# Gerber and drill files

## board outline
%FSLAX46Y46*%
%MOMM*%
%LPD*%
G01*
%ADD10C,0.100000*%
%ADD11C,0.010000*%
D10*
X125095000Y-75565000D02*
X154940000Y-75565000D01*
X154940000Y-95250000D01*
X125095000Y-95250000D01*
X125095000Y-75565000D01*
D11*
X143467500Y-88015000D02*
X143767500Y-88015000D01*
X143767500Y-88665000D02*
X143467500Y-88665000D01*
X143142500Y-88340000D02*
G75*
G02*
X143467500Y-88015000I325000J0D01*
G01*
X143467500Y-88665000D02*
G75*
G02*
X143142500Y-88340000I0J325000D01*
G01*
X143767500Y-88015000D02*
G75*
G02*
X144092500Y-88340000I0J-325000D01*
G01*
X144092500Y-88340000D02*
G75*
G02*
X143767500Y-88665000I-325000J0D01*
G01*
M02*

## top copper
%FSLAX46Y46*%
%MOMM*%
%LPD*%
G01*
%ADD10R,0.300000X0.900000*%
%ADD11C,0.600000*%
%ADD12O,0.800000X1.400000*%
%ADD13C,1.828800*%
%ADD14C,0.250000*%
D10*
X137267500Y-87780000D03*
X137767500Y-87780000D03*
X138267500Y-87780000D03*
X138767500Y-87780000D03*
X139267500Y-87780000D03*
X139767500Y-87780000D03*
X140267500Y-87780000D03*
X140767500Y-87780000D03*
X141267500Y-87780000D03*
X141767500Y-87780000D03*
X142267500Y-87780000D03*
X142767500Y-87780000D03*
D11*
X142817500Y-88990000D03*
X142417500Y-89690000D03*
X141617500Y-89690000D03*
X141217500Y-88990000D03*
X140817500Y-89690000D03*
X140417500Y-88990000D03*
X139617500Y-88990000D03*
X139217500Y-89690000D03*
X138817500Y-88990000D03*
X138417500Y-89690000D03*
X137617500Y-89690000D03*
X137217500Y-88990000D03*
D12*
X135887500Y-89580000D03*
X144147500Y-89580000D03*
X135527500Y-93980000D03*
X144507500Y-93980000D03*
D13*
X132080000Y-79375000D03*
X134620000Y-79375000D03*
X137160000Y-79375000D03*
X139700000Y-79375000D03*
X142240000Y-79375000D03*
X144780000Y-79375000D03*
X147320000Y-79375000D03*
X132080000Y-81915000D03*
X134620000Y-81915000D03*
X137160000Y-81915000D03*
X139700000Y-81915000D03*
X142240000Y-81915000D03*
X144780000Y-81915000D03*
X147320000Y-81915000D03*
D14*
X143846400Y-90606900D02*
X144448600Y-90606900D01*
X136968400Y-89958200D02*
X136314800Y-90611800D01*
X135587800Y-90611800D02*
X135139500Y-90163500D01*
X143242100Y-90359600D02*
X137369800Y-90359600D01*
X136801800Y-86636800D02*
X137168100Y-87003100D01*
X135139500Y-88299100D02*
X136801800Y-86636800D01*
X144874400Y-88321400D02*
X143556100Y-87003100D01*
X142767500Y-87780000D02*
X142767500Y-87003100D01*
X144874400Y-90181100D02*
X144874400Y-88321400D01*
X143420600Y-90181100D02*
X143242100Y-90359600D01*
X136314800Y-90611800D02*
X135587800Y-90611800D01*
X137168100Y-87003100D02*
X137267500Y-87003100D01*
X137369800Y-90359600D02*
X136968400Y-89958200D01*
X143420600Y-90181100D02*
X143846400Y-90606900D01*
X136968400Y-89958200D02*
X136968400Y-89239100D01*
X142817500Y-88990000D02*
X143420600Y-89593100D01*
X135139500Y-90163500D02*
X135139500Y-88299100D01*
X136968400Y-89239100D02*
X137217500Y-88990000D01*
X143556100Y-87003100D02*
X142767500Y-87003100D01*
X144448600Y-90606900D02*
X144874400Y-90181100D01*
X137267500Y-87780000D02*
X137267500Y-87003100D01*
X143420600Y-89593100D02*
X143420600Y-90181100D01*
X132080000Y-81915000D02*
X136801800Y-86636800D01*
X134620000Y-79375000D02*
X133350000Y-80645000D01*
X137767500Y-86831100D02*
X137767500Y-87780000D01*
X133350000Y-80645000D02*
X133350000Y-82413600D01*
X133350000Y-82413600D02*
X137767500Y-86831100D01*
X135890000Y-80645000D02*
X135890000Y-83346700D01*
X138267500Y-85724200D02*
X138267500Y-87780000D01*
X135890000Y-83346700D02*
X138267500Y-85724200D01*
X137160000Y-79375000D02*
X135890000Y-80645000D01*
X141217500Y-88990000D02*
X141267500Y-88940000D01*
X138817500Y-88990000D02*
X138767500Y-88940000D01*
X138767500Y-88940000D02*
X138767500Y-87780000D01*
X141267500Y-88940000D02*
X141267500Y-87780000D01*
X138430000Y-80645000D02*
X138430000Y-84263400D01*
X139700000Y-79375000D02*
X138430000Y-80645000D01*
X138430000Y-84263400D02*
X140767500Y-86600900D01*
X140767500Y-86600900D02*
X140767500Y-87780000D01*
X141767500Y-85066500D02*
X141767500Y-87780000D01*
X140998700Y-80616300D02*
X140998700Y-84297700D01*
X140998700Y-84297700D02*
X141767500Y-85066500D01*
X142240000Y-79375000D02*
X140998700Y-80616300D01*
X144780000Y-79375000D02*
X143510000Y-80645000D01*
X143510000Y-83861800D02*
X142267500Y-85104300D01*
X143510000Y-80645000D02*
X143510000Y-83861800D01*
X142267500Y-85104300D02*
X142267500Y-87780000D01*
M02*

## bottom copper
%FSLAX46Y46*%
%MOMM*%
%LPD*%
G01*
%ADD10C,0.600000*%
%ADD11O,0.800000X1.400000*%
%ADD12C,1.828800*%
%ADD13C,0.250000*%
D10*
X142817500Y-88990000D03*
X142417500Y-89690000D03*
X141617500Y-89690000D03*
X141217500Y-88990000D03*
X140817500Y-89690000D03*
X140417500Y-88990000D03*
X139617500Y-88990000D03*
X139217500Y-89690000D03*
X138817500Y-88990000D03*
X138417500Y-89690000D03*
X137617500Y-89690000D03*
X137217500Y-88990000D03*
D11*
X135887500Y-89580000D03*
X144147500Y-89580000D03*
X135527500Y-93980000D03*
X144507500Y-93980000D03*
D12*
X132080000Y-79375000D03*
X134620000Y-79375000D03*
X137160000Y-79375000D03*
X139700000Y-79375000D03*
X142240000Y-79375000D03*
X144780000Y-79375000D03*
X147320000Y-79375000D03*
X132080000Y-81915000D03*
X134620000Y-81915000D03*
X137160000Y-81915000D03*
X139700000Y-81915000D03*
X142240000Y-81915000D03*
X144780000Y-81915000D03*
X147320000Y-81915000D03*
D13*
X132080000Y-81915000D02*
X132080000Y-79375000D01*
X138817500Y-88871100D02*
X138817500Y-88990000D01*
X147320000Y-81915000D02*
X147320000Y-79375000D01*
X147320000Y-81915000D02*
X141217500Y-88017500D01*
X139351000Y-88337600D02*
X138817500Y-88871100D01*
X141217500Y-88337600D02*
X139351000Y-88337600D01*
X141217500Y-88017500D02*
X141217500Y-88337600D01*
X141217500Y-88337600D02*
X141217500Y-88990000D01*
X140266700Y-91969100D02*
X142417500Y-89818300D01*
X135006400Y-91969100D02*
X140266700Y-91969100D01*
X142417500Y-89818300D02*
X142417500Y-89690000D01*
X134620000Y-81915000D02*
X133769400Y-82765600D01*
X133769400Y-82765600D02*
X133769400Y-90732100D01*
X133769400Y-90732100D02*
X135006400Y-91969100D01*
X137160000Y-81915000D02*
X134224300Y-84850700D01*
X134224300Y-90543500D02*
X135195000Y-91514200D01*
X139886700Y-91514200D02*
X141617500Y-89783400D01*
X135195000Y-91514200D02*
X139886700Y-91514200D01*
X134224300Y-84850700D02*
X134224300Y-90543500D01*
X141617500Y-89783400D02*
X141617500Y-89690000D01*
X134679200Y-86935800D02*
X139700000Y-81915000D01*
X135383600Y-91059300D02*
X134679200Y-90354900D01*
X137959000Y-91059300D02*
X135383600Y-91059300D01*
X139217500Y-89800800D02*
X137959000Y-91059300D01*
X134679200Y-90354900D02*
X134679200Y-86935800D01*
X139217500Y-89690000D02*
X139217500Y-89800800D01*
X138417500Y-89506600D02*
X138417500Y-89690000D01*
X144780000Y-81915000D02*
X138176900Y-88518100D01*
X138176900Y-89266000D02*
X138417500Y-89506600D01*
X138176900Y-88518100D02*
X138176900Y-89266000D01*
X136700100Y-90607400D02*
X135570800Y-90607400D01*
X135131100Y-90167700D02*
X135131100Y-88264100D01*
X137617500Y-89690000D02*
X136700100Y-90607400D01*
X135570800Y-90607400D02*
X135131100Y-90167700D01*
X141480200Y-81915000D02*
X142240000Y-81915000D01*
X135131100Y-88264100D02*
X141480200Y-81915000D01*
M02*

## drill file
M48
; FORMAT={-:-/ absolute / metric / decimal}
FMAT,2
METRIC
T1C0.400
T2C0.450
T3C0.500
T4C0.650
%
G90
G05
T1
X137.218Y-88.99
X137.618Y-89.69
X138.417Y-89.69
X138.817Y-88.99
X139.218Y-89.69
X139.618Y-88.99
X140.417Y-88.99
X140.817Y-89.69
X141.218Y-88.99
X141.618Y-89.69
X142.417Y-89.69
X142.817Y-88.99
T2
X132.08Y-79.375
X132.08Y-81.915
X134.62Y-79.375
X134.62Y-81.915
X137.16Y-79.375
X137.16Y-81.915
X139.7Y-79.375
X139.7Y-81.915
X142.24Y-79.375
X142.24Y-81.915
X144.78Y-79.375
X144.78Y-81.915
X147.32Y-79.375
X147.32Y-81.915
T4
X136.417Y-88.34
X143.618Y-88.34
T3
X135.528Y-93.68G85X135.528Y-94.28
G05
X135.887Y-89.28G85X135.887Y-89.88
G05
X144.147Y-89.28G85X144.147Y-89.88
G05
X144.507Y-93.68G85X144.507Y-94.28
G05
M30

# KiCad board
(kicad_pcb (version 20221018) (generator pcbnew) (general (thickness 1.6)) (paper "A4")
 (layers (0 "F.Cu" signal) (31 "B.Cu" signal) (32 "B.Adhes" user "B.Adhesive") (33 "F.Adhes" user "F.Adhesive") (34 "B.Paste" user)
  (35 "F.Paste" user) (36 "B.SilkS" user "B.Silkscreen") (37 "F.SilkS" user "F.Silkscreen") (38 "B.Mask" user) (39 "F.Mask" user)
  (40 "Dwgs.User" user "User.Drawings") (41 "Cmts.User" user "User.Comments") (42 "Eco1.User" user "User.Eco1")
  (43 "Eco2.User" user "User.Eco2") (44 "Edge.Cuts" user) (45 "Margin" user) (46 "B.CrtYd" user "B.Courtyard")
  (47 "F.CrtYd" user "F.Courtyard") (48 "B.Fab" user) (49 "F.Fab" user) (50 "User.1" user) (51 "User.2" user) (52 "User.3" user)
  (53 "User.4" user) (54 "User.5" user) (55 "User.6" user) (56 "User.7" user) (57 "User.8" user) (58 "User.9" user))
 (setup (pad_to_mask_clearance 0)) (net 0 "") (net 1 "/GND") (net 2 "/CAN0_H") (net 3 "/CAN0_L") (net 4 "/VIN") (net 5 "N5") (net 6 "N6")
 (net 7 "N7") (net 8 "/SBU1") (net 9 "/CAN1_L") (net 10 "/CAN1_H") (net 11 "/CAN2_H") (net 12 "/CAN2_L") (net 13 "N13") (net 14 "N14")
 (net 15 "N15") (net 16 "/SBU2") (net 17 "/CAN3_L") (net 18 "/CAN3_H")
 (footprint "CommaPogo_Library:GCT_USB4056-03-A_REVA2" (layer "F.Cu") (at 140.0175 93.98)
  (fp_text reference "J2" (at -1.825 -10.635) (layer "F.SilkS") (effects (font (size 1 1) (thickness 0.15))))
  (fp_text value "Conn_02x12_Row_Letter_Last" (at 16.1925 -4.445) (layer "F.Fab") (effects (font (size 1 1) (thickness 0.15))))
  (fp_line (start 3.45 -5.965) (end 3.75 -5.965) (stroke (width 0.01) (type solid)) (layer "Edge.Cuts"))
  (fp_line (start 3.75 -5.315) (end 3.45 -5.315) (stroke (width 0.01) (type solid)) (layer "Edge.Cuts"))
  (fp_arc (start 3.125 -5.64) (mid 3.22019 -5.86981) (end 3.45 -5.965) (stroke (width 0.01) (type solid)) (layer "Edge.Cuts"))
  (fp_arc (start 3.45 -5.315) (mid 3.22019 -5.41019) (end 3.125 -5.64) (stroke (width 0.01) (type solid)) (layer "Edge.Cuts"))
  (fp_arc (start 3.75 -5.965) (mid 3.97981 -5.86981) (end 4.075 -5.64) (stroke (width 0.01) (type solid)) (layer "Edge.Cuts"))
  (fp_arc (start 4.075 -5.64) (mid 3.97981 -5.41019) (end 3.75 -5.315) (stroke (width 0.01) (type solid)) (layer "Edge.Cuts"))
  (pad "" np_thru_hole circle (at -3.6 -5.64) (size 0.65 0.65) (drill 0.65) (layers "*.Cu" "*.Mask"))
  (pad "" np_thru_hole circle (at 3.6 -5.64) (size 0.65 0.65) (drill 0.65) (layers "*.Cu" "*.Mask"))
  (pad "A1" smd rect (at -2.75 -6.2) (size 0.3 0.9) (layers "F.Cu" "F.Paste" "F.Mask") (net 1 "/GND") (solder_mask_margin 0.102))
  (pad "A2" smd rect (at -2.25 -6.2) (size 0.3 0.9) (layers "F.Cu" "F.Paste" "F.Mask") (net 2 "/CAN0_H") (solder_mask_margin 0.102))
  (pad "A3" smd rect (at -1.75 -6.2) (size 0.3 0.9) (layers "F.Cu" "F.Paste" "F.Mask") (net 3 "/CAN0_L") (solder_mask_margin 0.102))
  (pad "A4" smd rect (at -1.25 -6.2) (size 0.3 0.9) (layers "F.Cu" "F.Paste" "F.Mask") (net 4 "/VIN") (solder_mask_margin 0.102))
  (pad "A5" smd rect (at -0.75 -6.2) (size 0.3 0.9) (layers "F.Cu" "F.Paste" "F.Mask") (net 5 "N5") (solder_mask_margin 0.102))
  (pad "A6" smd rect (at -0.25 -6.2) (size 0.3 0.9) (layers "F.Cu" "F.Paste" "F.Mask") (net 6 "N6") (solder_mask_margin 0.102))
  (pad "A7" smd rect (at 0.25 -6.2) (size 0.3 0.9) (layers "F.Cu" "F.Paste" "F.Mask") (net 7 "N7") (solder_mask_margin 0.102))
  (pad "A8" smd rect (at 0.75 -6.2) (size 0.3 0.9) (layers "F.Cu" "F.Paste" "F.Mask") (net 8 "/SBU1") (solder_mask_margin 0.102))
  (pad "A9" smd rect (at 1.25 -6.2) (size 0.3 0.9) (layers "F.Cu" "F.Paste" "F.Mask") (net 4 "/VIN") (solder_mask_margin 0.102))
  (pad "A10" smd rect (at 1.75 -6.2) (size 0.3 0.9) (layers "F.Cu" "F.Paste" "F.Mask") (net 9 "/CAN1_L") (solder_mask_margin 0.102))
  (pad "A11" smd rect (at 2.25 -6.2) (size 0.3 0.9) (layers "F.Cu" "F.Paste" "F.Mask") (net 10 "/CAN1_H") (solder_mask_margin 0.102))
  (pad "A12" smd rect (at 2.75 -6.2) (size 0.3 0.9) (layers "F.Cu" "F.Paste" "F.Mask") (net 1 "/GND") (solder_mask_margin 0.102))
  (pad "B1" thru_hole circle (at 2.8 -4.99) (size 0.6 0.6) (drill 0.4) (layers "*.Cu" "*.Mask") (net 1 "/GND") (solder_mask_margin 0.102))
  (pad "B2" thru_hole circle (at 2.4 -4.29) (size 0.6 0.6) (drill 0.4) (layers "*.Cu" "*.Mask") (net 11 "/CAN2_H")
   (solder_mask_margin 0.102))
  (pad "B3" thru_hole circle (at 1.6 -4.29) (size 0.6 0.6) (drill 0.4) (layers "*.Cu" "*.Mask") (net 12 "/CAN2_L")
   (solder_mask_margin 0.102))
  (pad "B4" thru_hole circle (at 1.2 -4.99) (size 0.6 0.6) (drill 0.4) (layers "*.Cu" "*.Mask") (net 4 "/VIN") (solder_mask_margin 0.102))
  (pad "B5" thru_hole circle (at 0.8 -4.29) (size 0.6 0.6) (drill 0.4) (layers "*.Cu" "*.Mask") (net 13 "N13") (solder_mask_margin 0.102))
  (pad "B6" thru_hole circle (at 0.4 -4.99) (size 0.6 0.6) (drill 0.4) (layers "*.Cu" "*.Mask") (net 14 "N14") (solder_mask_margin 0.102))
  (pad "B7" thru_hole circle (at -0.4 -4.99) (size 0.6 0.6) (drill 0.4) (layers "*.Cu" "*.Mask") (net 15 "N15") (solder_mask_margin 0.102))
  (pad "B8" thru_hole circle (at -0.8 -4.29) (size 0.6 0.6) (drill 0.4) (layers "*.Cu" "*.Mask") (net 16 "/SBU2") (solder_mask_margin 0.102))
  (pad "B9" thru_hole circle (at -1.2 -4.99) (size 0.6 0.6) (drill 0.4) (layers "*.Cu" "*.Mask") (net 4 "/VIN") (solder_mask_margin 0.102))
  (pad "B10" thru_hole circle (at -1.6 -4.29) (size 0.6 0.6) (drill 0.4) (layers "*.Cu" "*.Mask") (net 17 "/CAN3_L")
   (solder_mask_margin 0.102))
  (pad "B11" thru_hole circle (at -2.4 -4.29) (size 0.6 0.6) (drill 0.4) (layers "*.Cu" "*.Mask") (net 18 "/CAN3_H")
   (solder_mask_margin 0.102))
  (pad "B12" thru_hole circle (at -2.8 -4.99) (size 0.6 0.6) (drill 0.4) (layers "*.Cu" "*.Mask") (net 1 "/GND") (solder_mask_margin 0.102))
  (pad "S1" thru_hole oval (at -4.13 -4.4) (size 0.8 1.4) (drill oval 0.5 1.1) (layers "*.Cu" "*.Mask") (solder_mask_margin 0.102))
  (pad "S2" thru_hole oval (at 4.13 -4.4) (size 0.8 1.4) (drill oval 0.5 1.1) (layers "*.Cu" "*.Mask") (solder_mask_margin 0.102))
  (pad "S3" thru_hole oval (at -4.49 0) (size 0.8 1.4) (drill oval 0.5 1.1) (layers "*.Cu" "*.Mask") (solder_mask_margin 0.102))
  (pad "S4" thru_hole oval (at 4.49 0) (size 0.8 1.4) (drill oval 0.5 1.1) (layers "*.Cu" "*.Mask") (solder_mask_margin 0.102)))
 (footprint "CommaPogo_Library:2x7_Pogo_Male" (layer "F.Cu") (at 139.7 83.82)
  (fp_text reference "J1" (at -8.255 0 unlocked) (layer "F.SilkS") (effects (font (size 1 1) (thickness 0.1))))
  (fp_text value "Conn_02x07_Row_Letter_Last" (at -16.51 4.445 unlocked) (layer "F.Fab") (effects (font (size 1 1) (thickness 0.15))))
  (pad "1" thru_hole circle (at -7.62 -4.445) (size 1.8288 1.8288) (drill 0.45) (layers "*.Cu" "*.Mask") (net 1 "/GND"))
  (pad "2" thru_hole circle (at -5.08 -4.445) (size 1.8288 1.8288) (drill 0.45) (layers "*.Cu" "*.Mask") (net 2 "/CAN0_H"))
  (pad "3" thru_hole circle (at -2.54 -4.445) (size 1.8288 1.8288) (drill 0.45) (layers "*.Cu" "*.Mask") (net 3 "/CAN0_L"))
  (pad "4" thru_hole circle (at 0 -4.445) (size 1.8288 1.8288) (drill 0.45) (layers "*.Cu" "*.Mask") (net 8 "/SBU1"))
  (pad "5" thru_hole circle (at 2.54 -4.445) (size 1.8288 1.8288) (drill 0.45) (layers "*.Cu" "*.Mask") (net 9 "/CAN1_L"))
  (pad "6" thru_hole circle (at 5.08 -4.445) (size 1.8288 1.8288) (drill 0.45) (layers "*.Cu" "*.Mask") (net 10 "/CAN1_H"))
  (pad "7" thru_hole circle (at 7.62 -4.445) (size 1.8288 1.8288) (drill 0.45) (layers "*.Cu" "*.Mask") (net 4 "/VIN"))
  (pad "8" thru_hole circle (at -7.62 -1.905) (size 1.8288 1.8288) (drill 0.45) (layers "*.Cu" "*.Mask") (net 1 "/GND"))
  (pad "9" thru_hole circle (at -5.08 -1.905) (size 1.8288 1.8288) (drill 0.45) (layers "*.Cu" "*.Mask") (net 11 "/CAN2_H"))
  (pad "10" thru_hole circle (at -2.54 -1.905) (size 1.8288 1.8288) (drill 0.45) (layers "*.Cu" "*.Mask") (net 12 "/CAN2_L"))
  (pad "11" thru_hole circle (at 0 -1.905) (size 1.8288 1.8288) (drill 0.45) (layers "*.Cu" "*.Mask") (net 16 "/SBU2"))
  (pad "12" thru_hole circle (at 2.54 -1.905) (size 1.8288 1.8288) (drill 0.45) (layers "*.Cu" "*.Mask") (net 18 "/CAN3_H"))
  (pad "13" thru_hole circle (at 5.08 -1.905) (size 1.8288 1.8288) (drill 0.45) (layers "*.Cu" "*.Mask") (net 17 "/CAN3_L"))
  (pad "14" thru_hole circle (at 7.62 -1.905) (size 1.8288 1.8288) (drill 0.45) (layers "*.Cu" "*.Mask") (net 4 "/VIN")))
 (gr_rect (start 125.095 75.565) (end 154.94 95.25) (stroke (width 0.1) (type default)) (fill none) (layer "Edge.Cuts"))
 (segment (start 143.8464 90.6069) (end 144.4486 90.6069) (width 0.25) (layer "F.Cu") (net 1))
 (segment (start 136.9684 89.9582) (end 136.3148 90.6118) (width 0.25) (layer "F.Cu") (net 1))
 (segment (start 135.5878 90.6118) (end 135.1395 90.1635) (width 0.25) (layer "F.Cu") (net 1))
 (segment (start 143.2421 90.3596) (end 137.3698 90.3596) (width 0.25) (layer "F.Cu") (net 1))
 (segment (start 136.8018 86.6368) (end 137.1681 87.0031) (width 0.25) (layer "F.Cu") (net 1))
 (segment (start 135.1395 88.2991) (end 136.8018 86.6368) (width 0.25) (layer "F.Cu") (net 1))
 (segment (start 144.8744 88.3214) (end 143.5561 87.0031) (width 0.25) (layer "F.Cu") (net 1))
 (segment (start 142.7675 87.78) (end 142.7675 87.0031) (width 0.25) (layer "F.Cu") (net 1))
 (segment (start 144.8744 90.1811) (end 144.8744 88.3214) (width 0.25) (layer "F.Cu") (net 1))
 (segment (start 143.4206 90.1811) (end 143.2421 90.3596) (width 0.25) (layer "F.Cu") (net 1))
 (segment (start 136.3148 90.6118) (end 135.5878 90.6118) (width 0.25) (layer "F.Cu") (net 1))
 (segment (start 137.1681 87.0031) (end 137.2675 87.0031) (width 0.25) (layer "F.Cu") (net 1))
 (segment (start 137.3698 90.3596) (end 136.9684 89.9582) (width 0.25) (layer "F.Cu") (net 1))
 (segment (start 143.4206 90.1811) (end 143.8464 90.6069) (width 0.25) (layer "F.Cu") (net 1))
 (segment (start 136.9684 89.9582) (end 136.9684 89.2391) (width 0.25) (layer "F.Cu") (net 1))
 (segment (start 142.8175 88.99) (end 143.4206 89.5931) (width 0.25) (layer "F.Cu") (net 1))
 (segment (start 135.1395 90.1635) (end 135.1395 88.2991) (width 0.25) (layer "F.Cu") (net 1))
 (segment (start 136.9684 89.2391) (end 137.2175 88.99) (width 0.25) (layer "F.Cu") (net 1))
 (segment (start 143.5561 87.0031) (end 142.7675 87.0031) (width 0.25) (layer "F.Cu") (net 1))
 (segment (start 144.4486 90.6069) (end 144.8744 90.1811) (width 0.25) (layer "F.Cu") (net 1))
 (segment (start 137.2675 87.78) (end 137.2675 87.0031) (width 0.25) (layer "F.Cu") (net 1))
 (segment (start 143.4206 89.5931) (end 143.4206 90.1811) (width 0.25) (layer "F.Cu") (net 1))
 (segment (start 132.08 81.915) (end 136.8018 86.6368) (width 0.25) (layer "F.Cu") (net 1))
 (segment (start 132.08 81.915) (end 132.08 79.375) (width 0.25) (layer "B.Cu") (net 1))
 (segment (start 134.62 79.375) (end 133.35 80.645) (width 0.25) (layer "F.Cu") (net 2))
 (segment (start 137.7675 86.8311) (end 137.7675 87.78) (width 0.25) (layer "F.Cu") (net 2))
 (segment (start 133.35 80.645) (end 133.35 82.4136) (width 0.25) (layer "F.Cu") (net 2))
 (segment (start 133.35 82.4136) (end 137.7675 86.8311) (width 0.25) (layer "F.Cu") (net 2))
 (segment (start 135.89 80.645) (end 135.89 83.3467) (width 0.25) (layer "F.Cu") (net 3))
 (segment (start 138.2675 85.7242) (end 138.2675 87.78) (width 0.25) (layer "F.Cu") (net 3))
 (segment (start 135.89 83.3467) (end 138.2675 85.7242) (width 0.25) (layer "F.Cu") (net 3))
 (segment (start 137.16 79.375) (end 135.89 80.645) (width 0.25) (layer "F.Cu") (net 3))
 (segment (start 141.2175 88.99) (end 141.2675 88.94) (width 0.25) (layer "F.Cu") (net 4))
 (segment (start 138.8175 88.99) (end 138.7675 88.94) (width 0.25) (layer "F.Cu") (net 4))
 (segment (start 138.7675 88.94) (end 138.7675 87.78) (width 0.25) (layer "F.Cu") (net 4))
 (segment (start 141.2675 88.94) (end 141.2675 87.78) (width 0.25) (layer "F.Cu") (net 4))
 (segment (start 138.8175 88.8711) (end 138.8175 88.99) (width 0.25) (layer "B.Cu") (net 4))
 (segment (start 147.32 81.915) (end 147.32 79.375) (width 0.25) (layer "B.Cu") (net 4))
 (segment (start 147.32 81.915) (end 141.2175 88.0175) (width 0.25) (layer "B.Cu") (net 4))
 (segment (start 139.351 88.3376) (end 138.8175 88.8711) (width 0.25) (layer "B.Cu") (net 4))
 (segment (start 141.2175 88.3376) (end 139.351 88.3376) (width 0.25) (layer "B.Cu") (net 4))
 (segment (start 141.2175 88.0175) (end 141.2175 88.3376) (width 0.25) (layer "B.Cu") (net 4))
 (segment (start 141.2175 88.3376) (end 141.2175 88.99) (width 0.25) (layer "B.Cu") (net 4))
 (segment (start 138.43 80.645) (end 138.43 84.2634) (width 0.25) (layer "F.Cu") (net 8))
 (segment (start 139.7 79.375) (end 138.43 80.645) (width 0.25) (layer "F.Cu") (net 8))
 (segment (start 138.43 84.2634) (end 140.7675 86.6009) (width 0.25) (layer "F.Cu") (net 8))
 (segment (start 140.7675 86.6009) (end 140.7675 87.78) (width 0.25) (layer "F.Cu") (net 8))
 (segment (start 141.7675 85.0665) (end 141.7675 87.78) (width 0.25) (layer "F.Cu") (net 9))
 (segment (start 140.9987 80.6163) (end 140.9987 84.2977) (width 0.25) (layer "F.Cu") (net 9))
 (segment (start 140.9987 84.2977) (end 141.7675 85.0665) (width 0.25) (layer "F.Cu") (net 9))
 (segment (start 142.24 79.375) (end 140.9987 80.6163) (width 0.25) (layer "F.Cu") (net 9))
 (segment (start 144.78 79.375) (end 143.51 80.645) (width 0.25) (layer "F.Cu") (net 10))
 (segment (start 143.51 83.8618) (end 142.2675 85.1043) (width 0.25) (layer "F.Cu") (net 10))
 (segment (start 143.51 80.645) (end 143.51 83.8618) (width 0.25) (layer "F.Cu") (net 10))
 (segment (start 142.2675 85.1043) (end 142.2675 87.78) (width 0.25) (layer "F.Cu") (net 10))
 (segment (start 140.2667 91.9691) (end 142.4175 89.8183) (width 0.25) (layer "B.Cu") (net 11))
 (segment (start 135.0064 91.9691) (end 140.2667 91.9691) (width 0.25) (layer "B.Cu") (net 11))
 (segment (start 142.4175 89.8183) (end 142.4175 89.69) (width 0.25) (layer "B.Cu") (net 11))
 (segment (start 134.62 81.915) (end 133.7694 82.7656) (width 0.25) (layer "B.Cu") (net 11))
 (segment (start 133.7694 82.7656) (end 133.7694 90.7321) (width 0.25) (layer "B.Cu") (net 11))
 (segment (start 133.7694 90.7321) (end 135.0064 91.9691) (width 0.25) (layer "B.Cu") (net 11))
 (segment (start 137.16 81.915) (end 134.2243 84.8507) (width 0.25) (layer "B.Cu") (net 12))
 (segment (start 134.2243 90.5435) (end 135.195 91.5142) (width 0.25) (layer "B.Cu") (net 12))
 (segment (start 139.8867 91.5142) (end 141.6175 89.7834) (width 0.25) (layer "B.Cu") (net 12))
 (segment (start 135.195 91.5142) (end 139.8867 91.5142) (width 0.25) (layer "B.Cu") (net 12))
 (segment (start 134.2243 84.8507) (end 134.2243 90.5435) (width 0.25) (layer "B.Cu") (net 12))
 (segment (start 141.6175 89.7834) (end 141.6175 89.69) (width 0.25) (layer "B.Cu") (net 12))
 (segment (start 134.6792 86.9358) (end 139.7 81.915) (width 0.25) (layer "B.Cu") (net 16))
 (segment (start 135.3836 91.0593) (end 134.6792 90.3549) (width 0.25) (layer "B.Cu") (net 16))
 (segment (start 137.959 91.0593) (end 135.3836 91.0593) (width 0.25) (layer "B.Cu") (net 16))
 (segment (start 139.2175 89.8008) (end 137.959 91.0593) (width 0.25) (layer "B.Cu") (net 16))
 (segment (start 134.6792 90.3549) (end 134.6792 86.9358) (width 0.25) (layer "B.Cu") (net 16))
 (segment (start 139.2175 89.69) (end 139.2175 89.8008) (width 0.25) (layer "B.Cu") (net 16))
 (segment (start 138.4175 89.5066) (end 138.4175 89.69) (width 0.25) (layer "B.Cu") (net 17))
 (segment (start 144.78 81.915) (end 138.1769 88.5181) (width 0.25) (layer "B.Cu") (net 17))
 (segment (start 138.1769 89.266) (end 138.4175 89.5066) (width 0.25) (layer "B.Cu") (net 17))
 (segment (start 138.1769 88.5181) (end 138.1769 89.266) (width 0.25) (layer "B.Cu") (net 17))
 (segment (start 136.7001 90.6074) (end 135.5708 90.6074) (width 0.25) (layer "B.Cu") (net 18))
 (segment (start 135.1311 90.1677) (end 135.1311 88.2641) (width 0.25) (layer "B.Cu") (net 18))
 (segment (start 137.6175 89.69) (end 136.7001 90.6074) (width 0.25) (layer "B.Cu") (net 18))
 (segment (start 135.5708 90.6074) (end 135.1311 90.1677) (width 0.25) (layer "B.Cu") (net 18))
 (segment (start 141.4802 81.915) (end 142.24 81.915) (width 0.25) (layer "B.Cu") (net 18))
 (segment (start 135.1311 88.2641) (end 141.4802 81.915) (width 0.25) (layer "B.Cu") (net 18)))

